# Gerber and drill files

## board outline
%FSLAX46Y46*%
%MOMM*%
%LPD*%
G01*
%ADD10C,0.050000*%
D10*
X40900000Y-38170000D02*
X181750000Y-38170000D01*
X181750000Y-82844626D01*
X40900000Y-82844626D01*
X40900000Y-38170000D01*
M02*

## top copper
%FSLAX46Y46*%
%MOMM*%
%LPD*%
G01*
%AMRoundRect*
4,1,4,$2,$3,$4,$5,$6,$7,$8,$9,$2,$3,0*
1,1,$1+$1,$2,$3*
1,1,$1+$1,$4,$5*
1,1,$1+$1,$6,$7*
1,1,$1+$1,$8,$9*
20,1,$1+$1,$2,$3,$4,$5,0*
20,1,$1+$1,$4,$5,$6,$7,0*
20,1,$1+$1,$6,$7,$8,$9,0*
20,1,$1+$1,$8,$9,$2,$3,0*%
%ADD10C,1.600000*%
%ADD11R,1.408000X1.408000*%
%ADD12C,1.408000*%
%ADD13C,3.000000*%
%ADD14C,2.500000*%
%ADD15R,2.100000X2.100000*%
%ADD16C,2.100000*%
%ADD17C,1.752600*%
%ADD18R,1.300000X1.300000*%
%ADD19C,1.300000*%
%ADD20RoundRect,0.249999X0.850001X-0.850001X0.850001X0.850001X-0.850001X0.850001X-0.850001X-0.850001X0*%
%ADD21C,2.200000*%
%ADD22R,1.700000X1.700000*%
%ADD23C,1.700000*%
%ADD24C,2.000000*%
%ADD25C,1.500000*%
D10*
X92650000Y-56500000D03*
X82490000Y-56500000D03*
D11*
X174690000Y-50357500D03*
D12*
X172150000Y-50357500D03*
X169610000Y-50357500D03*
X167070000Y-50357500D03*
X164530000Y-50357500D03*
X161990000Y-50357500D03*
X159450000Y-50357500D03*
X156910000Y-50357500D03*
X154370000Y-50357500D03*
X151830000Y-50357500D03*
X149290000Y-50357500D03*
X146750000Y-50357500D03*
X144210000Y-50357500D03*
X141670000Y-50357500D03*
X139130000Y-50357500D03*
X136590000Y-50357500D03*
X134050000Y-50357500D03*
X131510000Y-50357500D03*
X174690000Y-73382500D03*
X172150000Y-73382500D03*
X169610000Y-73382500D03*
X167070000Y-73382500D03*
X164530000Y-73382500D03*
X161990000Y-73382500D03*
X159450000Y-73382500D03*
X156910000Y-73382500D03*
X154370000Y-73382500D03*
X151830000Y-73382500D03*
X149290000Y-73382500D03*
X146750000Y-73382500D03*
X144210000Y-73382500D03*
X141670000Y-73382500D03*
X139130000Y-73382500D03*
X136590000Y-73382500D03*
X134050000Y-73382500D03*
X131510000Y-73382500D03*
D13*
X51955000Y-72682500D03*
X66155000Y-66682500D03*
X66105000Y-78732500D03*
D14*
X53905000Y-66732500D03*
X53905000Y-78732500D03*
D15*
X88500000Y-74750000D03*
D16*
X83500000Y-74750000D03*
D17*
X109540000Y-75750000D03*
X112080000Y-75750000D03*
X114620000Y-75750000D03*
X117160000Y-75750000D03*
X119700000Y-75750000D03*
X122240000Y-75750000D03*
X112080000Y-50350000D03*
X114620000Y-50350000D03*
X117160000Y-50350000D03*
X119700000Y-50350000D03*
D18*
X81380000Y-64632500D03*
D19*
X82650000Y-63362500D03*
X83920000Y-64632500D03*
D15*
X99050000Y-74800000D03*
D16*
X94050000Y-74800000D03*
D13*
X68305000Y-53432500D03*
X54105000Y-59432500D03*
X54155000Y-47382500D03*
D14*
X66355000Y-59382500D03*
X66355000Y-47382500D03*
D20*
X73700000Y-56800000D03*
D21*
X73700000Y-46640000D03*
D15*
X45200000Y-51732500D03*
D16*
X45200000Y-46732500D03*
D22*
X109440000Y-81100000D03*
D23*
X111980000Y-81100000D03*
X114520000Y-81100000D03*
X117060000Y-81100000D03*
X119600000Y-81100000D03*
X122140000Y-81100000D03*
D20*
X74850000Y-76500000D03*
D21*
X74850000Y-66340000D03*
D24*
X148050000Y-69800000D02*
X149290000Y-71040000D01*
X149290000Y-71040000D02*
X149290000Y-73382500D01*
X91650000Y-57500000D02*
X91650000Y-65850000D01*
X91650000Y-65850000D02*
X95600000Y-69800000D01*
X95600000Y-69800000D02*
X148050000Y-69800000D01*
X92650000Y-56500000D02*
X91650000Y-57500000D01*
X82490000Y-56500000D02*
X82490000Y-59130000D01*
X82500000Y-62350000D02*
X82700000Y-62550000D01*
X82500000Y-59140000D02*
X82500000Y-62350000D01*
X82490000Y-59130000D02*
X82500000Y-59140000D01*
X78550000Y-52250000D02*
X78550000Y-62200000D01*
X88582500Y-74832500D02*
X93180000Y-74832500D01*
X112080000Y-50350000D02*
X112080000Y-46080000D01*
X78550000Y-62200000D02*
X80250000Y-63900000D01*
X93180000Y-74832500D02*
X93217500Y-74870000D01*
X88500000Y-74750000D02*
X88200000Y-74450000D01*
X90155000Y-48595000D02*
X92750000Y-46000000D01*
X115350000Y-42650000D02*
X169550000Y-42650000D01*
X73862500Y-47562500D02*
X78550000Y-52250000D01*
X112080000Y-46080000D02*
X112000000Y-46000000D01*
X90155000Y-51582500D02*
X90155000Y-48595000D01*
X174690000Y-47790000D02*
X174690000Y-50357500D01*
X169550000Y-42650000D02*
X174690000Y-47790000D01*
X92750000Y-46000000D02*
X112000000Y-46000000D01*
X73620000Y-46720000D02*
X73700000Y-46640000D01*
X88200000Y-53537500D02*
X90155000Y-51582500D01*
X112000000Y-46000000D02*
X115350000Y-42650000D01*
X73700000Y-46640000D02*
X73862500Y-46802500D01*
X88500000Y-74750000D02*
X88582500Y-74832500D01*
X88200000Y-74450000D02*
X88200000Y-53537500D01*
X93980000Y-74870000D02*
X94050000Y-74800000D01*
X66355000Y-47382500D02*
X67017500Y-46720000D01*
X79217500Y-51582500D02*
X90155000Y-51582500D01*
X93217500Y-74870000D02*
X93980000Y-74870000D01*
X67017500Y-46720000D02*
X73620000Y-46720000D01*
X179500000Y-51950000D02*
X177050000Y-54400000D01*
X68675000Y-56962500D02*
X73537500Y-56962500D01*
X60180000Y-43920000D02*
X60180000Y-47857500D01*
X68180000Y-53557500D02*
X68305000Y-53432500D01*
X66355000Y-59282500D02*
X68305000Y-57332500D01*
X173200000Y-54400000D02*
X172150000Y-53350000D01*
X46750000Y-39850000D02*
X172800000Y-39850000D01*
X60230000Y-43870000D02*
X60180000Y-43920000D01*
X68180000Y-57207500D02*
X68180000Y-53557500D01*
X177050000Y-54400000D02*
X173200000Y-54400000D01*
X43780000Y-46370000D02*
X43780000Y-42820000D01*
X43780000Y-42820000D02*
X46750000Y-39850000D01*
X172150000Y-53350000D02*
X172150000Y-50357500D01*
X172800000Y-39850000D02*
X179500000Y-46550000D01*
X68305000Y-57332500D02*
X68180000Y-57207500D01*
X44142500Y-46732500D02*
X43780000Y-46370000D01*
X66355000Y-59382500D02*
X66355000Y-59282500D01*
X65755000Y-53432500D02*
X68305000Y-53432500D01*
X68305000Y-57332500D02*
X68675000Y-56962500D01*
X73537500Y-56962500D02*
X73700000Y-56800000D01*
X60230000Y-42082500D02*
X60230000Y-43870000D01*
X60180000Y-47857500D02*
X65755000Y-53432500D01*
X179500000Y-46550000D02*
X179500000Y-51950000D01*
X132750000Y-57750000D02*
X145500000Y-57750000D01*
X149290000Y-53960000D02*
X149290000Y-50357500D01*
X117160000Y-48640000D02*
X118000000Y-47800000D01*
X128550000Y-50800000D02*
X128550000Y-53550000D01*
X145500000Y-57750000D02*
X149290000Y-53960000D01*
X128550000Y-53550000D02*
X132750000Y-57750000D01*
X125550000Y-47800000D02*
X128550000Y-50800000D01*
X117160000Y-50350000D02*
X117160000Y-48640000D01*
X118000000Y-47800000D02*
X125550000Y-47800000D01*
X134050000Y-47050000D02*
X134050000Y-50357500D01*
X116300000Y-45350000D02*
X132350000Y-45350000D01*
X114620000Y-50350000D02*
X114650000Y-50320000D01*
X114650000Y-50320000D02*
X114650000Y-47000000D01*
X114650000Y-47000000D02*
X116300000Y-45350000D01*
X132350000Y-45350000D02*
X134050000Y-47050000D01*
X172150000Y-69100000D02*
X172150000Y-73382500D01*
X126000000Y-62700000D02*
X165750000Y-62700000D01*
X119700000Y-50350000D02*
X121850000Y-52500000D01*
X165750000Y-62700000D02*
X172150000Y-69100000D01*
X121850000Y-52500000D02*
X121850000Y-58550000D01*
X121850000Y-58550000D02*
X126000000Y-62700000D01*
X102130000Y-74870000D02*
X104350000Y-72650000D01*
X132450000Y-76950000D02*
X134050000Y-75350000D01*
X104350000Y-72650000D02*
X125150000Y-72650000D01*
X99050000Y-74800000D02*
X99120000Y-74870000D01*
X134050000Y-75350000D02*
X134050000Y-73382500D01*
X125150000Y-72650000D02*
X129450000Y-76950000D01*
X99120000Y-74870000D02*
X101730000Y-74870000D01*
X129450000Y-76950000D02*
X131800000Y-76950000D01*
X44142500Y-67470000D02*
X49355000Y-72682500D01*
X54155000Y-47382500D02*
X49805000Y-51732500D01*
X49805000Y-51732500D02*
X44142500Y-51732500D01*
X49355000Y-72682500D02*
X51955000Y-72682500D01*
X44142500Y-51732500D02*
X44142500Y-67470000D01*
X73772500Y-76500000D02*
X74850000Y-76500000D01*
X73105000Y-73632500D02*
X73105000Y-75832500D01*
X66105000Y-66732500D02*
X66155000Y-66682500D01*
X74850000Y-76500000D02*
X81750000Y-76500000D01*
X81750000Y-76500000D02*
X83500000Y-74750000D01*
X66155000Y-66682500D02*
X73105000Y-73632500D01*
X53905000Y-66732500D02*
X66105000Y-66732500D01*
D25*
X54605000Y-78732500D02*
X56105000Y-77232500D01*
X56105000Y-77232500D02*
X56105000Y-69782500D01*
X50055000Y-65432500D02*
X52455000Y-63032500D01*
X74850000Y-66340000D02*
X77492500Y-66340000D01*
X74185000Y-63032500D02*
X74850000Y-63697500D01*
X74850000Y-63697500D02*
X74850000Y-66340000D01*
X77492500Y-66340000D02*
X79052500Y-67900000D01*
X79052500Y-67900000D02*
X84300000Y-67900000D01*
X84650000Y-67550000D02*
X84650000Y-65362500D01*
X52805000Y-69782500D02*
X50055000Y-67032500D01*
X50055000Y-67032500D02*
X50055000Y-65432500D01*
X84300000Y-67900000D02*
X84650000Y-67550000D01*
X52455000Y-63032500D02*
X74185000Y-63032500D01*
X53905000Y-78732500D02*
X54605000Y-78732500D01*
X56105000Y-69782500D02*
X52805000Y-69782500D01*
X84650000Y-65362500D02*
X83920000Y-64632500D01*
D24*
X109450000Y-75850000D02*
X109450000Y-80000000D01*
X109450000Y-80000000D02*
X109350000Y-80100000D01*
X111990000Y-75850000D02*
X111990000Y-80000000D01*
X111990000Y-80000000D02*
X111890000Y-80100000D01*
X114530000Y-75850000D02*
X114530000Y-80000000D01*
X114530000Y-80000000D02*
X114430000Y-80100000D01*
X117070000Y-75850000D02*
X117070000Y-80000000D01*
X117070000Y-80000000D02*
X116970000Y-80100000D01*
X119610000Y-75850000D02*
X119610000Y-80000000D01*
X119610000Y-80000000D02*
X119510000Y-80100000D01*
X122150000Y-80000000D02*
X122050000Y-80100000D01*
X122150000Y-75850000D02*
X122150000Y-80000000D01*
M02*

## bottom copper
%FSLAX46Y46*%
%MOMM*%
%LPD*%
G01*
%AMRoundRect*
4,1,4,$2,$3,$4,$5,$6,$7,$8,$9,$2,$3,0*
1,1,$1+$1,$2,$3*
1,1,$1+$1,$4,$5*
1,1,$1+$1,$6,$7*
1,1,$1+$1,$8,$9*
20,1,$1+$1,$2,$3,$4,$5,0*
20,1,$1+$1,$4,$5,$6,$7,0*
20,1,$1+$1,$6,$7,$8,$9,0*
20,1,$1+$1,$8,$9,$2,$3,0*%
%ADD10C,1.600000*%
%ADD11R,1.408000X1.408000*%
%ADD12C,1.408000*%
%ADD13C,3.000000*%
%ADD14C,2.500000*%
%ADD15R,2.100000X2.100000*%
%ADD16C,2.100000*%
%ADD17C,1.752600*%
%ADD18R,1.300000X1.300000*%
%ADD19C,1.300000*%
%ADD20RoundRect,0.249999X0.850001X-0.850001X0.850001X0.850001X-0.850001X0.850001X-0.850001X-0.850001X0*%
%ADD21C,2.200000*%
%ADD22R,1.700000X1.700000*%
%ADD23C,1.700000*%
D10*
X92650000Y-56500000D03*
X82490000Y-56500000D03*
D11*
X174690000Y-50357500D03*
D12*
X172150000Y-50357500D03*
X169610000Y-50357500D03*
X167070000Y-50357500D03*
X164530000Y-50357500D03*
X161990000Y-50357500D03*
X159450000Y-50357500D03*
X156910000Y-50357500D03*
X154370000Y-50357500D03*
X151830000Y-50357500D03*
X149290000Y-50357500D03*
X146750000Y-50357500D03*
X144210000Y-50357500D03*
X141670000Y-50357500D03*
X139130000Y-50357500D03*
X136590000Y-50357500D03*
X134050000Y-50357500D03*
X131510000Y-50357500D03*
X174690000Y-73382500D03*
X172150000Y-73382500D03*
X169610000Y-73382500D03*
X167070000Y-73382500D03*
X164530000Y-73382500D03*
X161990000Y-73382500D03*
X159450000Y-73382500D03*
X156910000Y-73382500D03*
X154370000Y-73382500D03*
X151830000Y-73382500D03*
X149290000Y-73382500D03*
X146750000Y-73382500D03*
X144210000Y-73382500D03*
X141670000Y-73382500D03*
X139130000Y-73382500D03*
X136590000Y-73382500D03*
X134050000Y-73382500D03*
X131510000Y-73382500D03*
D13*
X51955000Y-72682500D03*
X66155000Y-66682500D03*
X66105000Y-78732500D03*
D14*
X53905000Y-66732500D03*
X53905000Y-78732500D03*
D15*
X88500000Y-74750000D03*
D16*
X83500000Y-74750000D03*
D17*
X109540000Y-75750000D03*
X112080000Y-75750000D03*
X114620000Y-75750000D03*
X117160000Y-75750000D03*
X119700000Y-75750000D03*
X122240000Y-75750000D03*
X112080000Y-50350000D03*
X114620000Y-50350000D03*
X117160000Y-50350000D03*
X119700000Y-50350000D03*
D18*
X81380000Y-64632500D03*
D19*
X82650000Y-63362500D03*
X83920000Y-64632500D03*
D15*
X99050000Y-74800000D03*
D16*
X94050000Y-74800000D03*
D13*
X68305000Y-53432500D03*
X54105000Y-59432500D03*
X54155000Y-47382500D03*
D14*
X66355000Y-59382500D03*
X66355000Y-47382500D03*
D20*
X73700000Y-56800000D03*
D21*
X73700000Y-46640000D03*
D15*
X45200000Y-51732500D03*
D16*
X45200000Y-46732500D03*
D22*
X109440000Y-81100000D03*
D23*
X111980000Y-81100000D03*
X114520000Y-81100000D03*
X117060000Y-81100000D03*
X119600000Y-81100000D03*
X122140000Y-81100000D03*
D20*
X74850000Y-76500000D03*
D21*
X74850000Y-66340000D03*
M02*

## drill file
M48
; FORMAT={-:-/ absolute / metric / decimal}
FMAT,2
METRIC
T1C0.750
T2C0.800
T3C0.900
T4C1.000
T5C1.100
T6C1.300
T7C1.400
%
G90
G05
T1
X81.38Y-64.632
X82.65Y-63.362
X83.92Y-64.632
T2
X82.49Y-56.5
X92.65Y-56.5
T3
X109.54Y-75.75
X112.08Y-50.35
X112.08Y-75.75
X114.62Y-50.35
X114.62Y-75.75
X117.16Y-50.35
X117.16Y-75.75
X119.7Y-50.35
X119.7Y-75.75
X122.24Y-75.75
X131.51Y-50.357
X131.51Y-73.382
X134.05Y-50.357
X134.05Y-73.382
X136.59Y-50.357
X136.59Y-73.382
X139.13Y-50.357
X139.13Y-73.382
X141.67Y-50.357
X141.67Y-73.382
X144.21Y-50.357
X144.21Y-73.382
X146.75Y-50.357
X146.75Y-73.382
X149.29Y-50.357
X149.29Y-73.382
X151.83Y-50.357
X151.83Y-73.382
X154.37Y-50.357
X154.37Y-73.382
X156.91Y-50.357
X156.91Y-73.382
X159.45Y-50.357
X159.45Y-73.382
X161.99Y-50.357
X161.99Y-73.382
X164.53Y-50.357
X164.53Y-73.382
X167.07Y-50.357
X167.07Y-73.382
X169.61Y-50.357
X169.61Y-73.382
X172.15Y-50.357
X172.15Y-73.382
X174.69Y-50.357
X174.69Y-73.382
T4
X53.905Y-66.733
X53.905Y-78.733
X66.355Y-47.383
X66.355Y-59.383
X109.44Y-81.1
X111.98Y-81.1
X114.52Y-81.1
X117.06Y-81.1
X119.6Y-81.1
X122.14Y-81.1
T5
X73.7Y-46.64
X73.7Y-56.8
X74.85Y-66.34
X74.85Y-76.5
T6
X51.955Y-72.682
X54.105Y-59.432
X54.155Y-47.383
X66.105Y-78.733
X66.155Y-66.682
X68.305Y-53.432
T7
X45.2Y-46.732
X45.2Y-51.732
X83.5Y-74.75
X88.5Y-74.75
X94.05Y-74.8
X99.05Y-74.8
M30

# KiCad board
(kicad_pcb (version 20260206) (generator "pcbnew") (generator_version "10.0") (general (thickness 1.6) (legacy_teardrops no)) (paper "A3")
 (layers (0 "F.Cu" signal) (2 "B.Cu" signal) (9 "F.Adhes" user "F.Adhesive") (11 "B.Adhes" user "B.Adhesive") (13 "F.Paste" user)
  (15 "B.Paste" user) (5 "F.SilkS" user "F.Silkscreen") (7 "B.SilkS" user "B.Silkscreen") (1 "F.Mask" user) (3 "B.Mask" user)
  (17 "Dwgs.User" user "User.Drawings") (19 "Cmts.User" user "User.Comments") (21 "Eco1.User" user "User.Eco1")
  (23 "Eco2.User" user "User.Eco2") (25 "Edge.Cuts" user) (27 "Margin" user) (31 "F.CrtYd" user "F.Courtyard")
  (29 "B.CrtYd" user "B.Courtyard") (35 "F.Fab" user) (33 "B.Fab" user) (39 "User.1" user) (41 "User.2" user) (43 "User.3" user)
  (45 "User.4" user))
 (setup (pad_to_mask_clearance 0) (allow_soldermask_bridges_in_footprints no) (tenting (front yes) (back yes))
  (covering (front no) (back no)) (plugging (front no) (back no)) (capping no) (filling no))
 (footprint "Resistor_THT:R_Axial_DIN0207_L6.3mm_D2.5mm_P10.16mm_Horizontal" (layer "F.Cu") (at 92.65 56.5 180)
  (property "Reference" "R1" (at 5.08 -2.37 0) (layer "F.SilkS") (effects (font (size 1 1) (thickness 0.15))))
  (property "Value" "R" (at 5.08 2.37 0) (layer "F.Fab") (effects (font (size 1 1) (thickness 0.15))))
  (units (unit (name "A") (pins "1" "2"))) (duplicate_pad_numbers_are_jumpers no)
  (pad "1" thru_hole circle (at 0 0 180) (size 1.6 1.6) (drill 0.8) (layers "*.Cu" "*.Mask") (remove_unused_layers no) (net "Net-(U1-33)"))
  (pad "2" thru_hole circle (at 10.16 0 180) (size 1.6 1.6) (drill 0.8) (layers "*.Cu" "*.Mask") (remove_unused_layers no)
   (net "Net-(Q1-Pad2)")))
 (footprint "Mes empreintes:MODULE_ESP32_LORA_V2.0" (layer "F.Cu") (at 152.31 61.87 180)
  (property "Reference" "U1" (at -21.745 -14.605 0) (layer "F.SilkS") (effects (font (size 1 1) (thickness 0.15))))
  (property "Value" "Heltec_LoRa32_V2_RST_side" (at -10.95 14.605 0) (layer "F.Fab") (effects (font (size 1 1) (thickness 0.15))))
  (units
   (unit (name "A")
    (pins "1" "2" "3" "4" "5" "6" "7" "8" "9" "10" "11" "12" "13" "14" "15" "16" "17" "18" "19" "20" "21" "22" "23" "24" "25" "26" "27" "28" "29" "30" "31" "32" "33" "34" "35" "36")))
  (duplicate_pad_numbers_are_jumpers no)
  (pad "1" thru_hole rect (at -22.38 11.5125 180) (size 1.408 1.408) (drill 0.9) (layers "*.Cu" "*.Mask") (remove_unused_layers no)
   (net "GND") (solder_mask_margin 0.102))
  (pad "2" thru_hole circle (at -19.84 11.5125 180) (size 1.408 1.408) (drill 0.9) (layers "*.Cu" "*.Mask") (remove_unused_layers no)
   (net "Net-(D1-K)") (solder_mask_margin 0.102))
  (pad "3" thru_hole circle (at -17.3 11.5125 180) (size 1.408 1.408) (drill 0.9) (layers "*.Cu" "*.Mask") (remove_unused_layers no)
   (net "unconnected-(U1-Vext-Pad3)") (solder_mask_margin 0.102))
  (pad "4" thru_hole circle (at -14.76 11.5125 180) (size 1.408 1.408) (drill 0.9) (layers "*.Cu" "*.Mask") (remove_unused_layers no)
   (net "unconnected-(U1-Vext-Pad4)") (solder_mask_margin 0.102))
  (pad "5" thru_hole circle (at -12.22 11.5125 180) (size 1.408 1.408) (drill 0.9) (layers "*.Cu" "*.Mask") (remove_unused_layers no)
   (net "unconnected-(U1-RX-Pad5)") (solder_mask_margin 0.102))
  (pad "6" thru_hole circle (at -9.68 11.5125 180) (size 1.408 1.408) (drill 0.9) (layers "*.Cu" "*.Mask") (remove_unused_layers no)
   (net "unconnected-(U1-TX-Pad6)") (solder_mask_margin 0.102))
  (pad "7" thru_hole circle (at -7.14 11.5125 180) (size 1.408 1.408) (drill 0.9) (layers "*.Cu" "*.Mask") (remove_unused_layers no)
   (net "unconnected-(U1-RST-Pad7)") (solder_mask_margin 0.102))
  (pad "8" thru_hole circle (at -4.6 11.5125 180) (size 1.408 1.408) (drill 0.9) (layers "*.Cu" "*.Mask") (remove_unused_layers no)
   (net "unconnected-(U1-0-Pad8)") (solder_mask_margin 0.102))
  (pad "9" thru_hole circle (at -2.06 11.5125 180) (size 1.408 1.408) (drill 0.9) (layers "*.Cu" "*.Mask") (remove_unused_layers no)
   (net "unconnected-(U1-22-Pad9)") (solder_mask_margin 0.102))
  (pad "10" thru_hole circle (at 0.48 11.5125 180) (size 1.408 1.408) (drill 0.9) (layers "*.Cu" "*.Mask") (remove_unused_layers no)
   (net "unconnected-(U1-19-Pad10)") (solder_mask_margin 0.102))
  (pad "11" thru_hole circle (at 3.02 11.5125 180) (size 1.408 1.408) (drill 0.9) (layers "*.Cu" "*.Mask") (remove_unused_layers no)
   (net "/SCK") (solder_mask_margin 0.102))
  (pad "12" thru_hole circle (at 5.56 11.5125 180) (size 1.408 1.408) (drill 0.9) (layers "*.Cu" "*.Mask") (remove_unused_layers no)
   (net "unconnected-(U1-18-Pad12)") (solder_mask_margin 0.102))
  (pad "13" thru_hole circle (at 8.1 11.5125 180) (size 1.408 1.408) (drill 0.9) (layers "*.Cu" "*.Mask") (remove_unused_layers no)
   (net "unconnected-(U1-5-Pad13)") (solder_mask_margin 0.102))
  (pad "14" thru_hole circle (at 10.64 11.5125 180) (size 1.408 1.408) (drill 0.9) (layers "*.Cu" "*.Mask") (remove_unused_layers no)
   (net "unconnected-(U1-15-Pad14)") (solder_mask_margin 0.102))
  (pad "15" thru_hole circle (at 13.18 11.5125 180) (size 1.408 1.408) (drill 0.9) (layers "*.Cu" "*.Mask") (remove_unused_layers no)
   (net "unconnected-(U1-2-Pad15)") (solder_mask_margin 0.102))
  (pad "16" thru_hole circle (at 15.72 11.5125 180) (size 1.408 1.408) (drill 0.9) (layers "*.Cu" "*.Mask") (remove_unused_layers no)
   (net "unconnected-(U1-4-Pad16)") (solder_mask_margin 0.102))
  (pad "17" thru_hole circle (at 18.26 11.5125 180) (size 1.408 1.408) (drill 0.9) (layers "*.Cu" "*.Mask") (remove_unused_layers no)
   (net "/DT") (solder_mask_margin 0.102))
  (pad "18" thru_hole circle (at 20.8 11.5125 180) (size 1.408 1.408) (drill 0.9) (layers "*.Cu" "*.Mask") (remove_unused_layers no)
   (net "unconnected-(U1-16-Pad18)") (solder_mask_margin 0.102))
  (pad "19" thru_hole circle (at -22.38 -11.5125 180) (size 1.408 1.408) (drill 0.9) (layers "*.Cu" "*.Mask") (remove_unused_layers no)
   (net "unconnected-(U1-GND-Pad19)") (solder_mask_margin 0.102))
  (pad "20" thru_hole circle (at -19.84 -11.5125 180) (size 1.408 1.408) (drill 0.9) (layers "*.Cu" "*.Mask") (remove_unused_layers no)
   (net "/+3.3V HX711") (solder_mask_margin 0.102))
  (pad "21" thru_hole circle (at -17.3 -11.5125 180) (size 1.408 1.408) (drill 0.9) (layers "*.Cu" "*.Mask") (remove_unused_layers no)
   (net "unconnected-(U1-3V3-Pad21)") (solder_mask_margin 0.102))
  (pad "22" thru_hole circle (at -14.76 -11.5125 180) (size 1.408 1.408) (drill 0.9) (layers "*.Cu" "*.Mask") (remove_unused_layers no)
   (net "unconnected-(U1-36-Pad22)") (solder_mask_margin 0.102))
  (pad "23" thru_hole circle (at -12.22 -11.5125 180) (size 1.408 1.408) (drill 0.9) (layers "*.Cu" "*.Mask") (remove_unused_layers no)
   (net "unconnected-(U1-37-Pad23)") (solder_mask_margin 0.102))
  (pad "24" thru_hole circle (at -9.68 -11.5125 180) (size 1.408 1.408) (drill 0.9) (layers "*.Cu" "*.Mask") (remove_unused_layers no)
   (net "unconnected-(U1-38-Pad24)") (solder_mask_margin 0.102))
  (pad "25" thru_hole circle (at -7.14 -11.5125 180) (size 1.408 1.408) (drill 0.9) (layers "*.Cu" "*.Mask") (remove_unused_layers no)
   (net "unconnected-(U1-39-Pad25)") (solder_mask_margin 0.102))
  (pad "26" thru_hole circle (at -4.6 -11.5125 180) (size 1.408 1.408) (drill 0.9) (layers "*.Cu" "*.Mask") (remove_unused_layers no)
   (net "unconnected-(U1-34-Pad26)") (solder_mask_margin 0.102))
  (pad "27" thru_hole circle (at -2.06 -11.5125 180) (size 1.408 1.408) (drill 0.9) (layers "*.Cu" "*.Mask") (remove_unused_layers no)
   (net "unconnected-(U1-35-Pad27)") (solder_mask_margin 0.102))
  (pad "28" thru_hole circle (at 0.48 -11.5125 180) (size 1.408 1.408) (drill 0.9) (layers "*.Cu" "*.Mask") (remove_unused_layers no)
   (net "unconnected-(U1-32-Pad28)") (solder_mask_margin 0.102))
  (pad "29" thru_hole circle (at 3.02 -11.5125 180) (size 1.408 1.408) (drill 0.9) (layers "*.Cu" "*.Mask") (remove_unused_layers no)
   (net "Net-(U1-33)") (solder_mask_margin 0.102))
  (pad "30" thru_hole circle (at 5.56 -11.5125 180) (size 1.408 1.408) (drill 0.9) (layers "*.Cu" "*.Mask") (remove_unused_layers no)
   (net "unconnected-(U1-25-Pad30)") (solder_mask_margin 0.102))
  (pad "31" thru_hole circle (at 8.1 -11.5125 180) (size 1.408 1.408) (drill 0.9) (layers "*.Cu" "*.Mask") (remove_unused_layers no)
   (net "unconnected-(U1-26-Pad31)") (solder_mask_margin 0.102))
  (pad "32" thru_hole circle (at 10.64 -11.5125 180) (size 1.408 1.408) (drill 0.9) (layers "*.Cu" "*.Mask") (remove_unused_layers no)
   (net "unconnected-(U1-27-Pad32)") (solder_mask_margin 0.102))
  (pad "33" thru_hole circle (at 13.18 -11.5125 180) (size 1.408 1.408) (drill 0.9) (layers "*.Cu" "*.Mask") (remove_unused_layers no)
   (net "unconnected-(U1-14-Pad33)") (solder_mask_margin 0.102))
  (pad "34" thru_hole circle (at 15.72 -11.5125 180) (size 1.408 1.408) (drill 0.9) (layers "*.Cu" "*.Mask") (remove_unused_layers no)
   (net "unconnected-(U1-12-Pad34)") (solder_mask_margin 0.102))
  (pad "35" thru_hole circle (at 18.26 -11.5125 180) (size 1.408 1.408) (drill 0.9) (layers "*.Cu" "*.Mask") (remove_unused_layers no)
   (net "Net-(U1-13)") (solder_mask_margin 0.102))
  (pad "36" thru_hole circle (at 20.8 -11.5125 180) (size 1.408 1.408) (drill 0.9) (layers "*.Cu" "*.Mask") (remove_unused_layers no)
   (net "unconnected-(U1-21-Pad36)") (solder_mask_margin 0.102)))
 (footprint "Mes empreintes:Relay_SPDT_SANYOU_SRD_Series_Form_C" (layer "F.Cu") (at 51.955 72.6825)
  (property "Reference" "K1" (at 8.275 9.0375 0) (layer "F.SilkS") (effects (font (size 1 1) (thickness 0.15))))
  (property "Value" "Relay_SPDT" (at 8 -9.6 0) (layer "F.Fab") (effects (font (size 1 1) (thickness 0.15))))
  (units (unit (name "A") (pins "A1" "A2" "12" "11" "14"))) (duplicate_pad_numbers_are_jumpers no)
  (pad "11" thru_hole circle (at 0 0 90) (size 3 3) (drill 1.3) (layers "*.Cu" "*.Mask") (remove_unused_layers no) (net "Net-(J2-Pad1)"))
  (pad "12" thru_hole circle (at 14.2 -6 90) (size 3 3) (drill 1.3) (layers "*.Cu" "*.Mask") (remove_unused_layers no) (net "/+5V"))
  (pad "14" thru_hole circle (at 14.15 6.05 90) (size 3 3) (drill 1.3) (layers "*.Cu" "*.Mask") (remove_unused_layers no)
   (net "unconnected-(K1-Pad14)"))
  (pad "A1" thru_hole circle (at 1.95 -5.95 90) (size 2.5 2.5) (drill 1) (layers "*.Cu" "*.Mask") (remove_unused_layers no) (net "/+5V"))
  (pad "A2" thru_hole circle (at 1.95 6.05 90) (size 2.5 2.5) (drill 1) (layers "*.Cu" "*.Mask") (remove_unused_layers no)
   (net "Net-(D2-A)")))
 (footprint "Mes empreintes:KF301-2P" (layer "F.Cu") (at 86 74.75 180)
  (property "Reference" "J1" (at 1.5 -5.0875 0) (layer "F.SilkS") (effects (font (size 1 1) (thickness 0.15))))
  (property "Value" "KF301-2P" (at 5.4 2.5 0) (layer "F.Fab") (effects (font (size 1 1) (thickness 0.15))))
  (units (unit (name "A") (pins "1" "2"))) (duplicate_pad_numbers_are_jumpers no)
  (pad "1" thru_hole rect (at -2.5 0 180) (size 2.1 2.1) (drill 1.4) (layers "*.Cu" "*.Mask") (remove_unused_layers no) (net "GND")
   (solder_mask_margin 0.102))
  (pad "2" thru_hole circle (at 2.5 0 180) (size 2.1 2.1) (drill 1.4) (layers "*.Cu" "*.Mask") (remove_unused_layers no) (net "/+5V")
   (solder_mask_margin 0.102)))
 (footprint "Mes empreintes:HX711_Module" (layer "F.Cu") (at 109.54 75.75 90)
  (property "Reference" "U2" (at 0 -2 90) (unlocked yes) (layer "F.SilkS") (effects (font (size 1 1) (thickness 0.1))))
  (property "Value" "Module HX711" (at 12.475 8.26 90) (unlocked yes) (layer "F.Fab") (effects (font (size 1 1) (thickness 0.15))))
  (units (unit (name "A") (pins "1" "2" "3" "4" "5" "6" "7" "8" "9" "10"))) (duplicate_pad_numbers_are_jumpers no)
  (pad "1" thru_hole circle (at 0 0 90) (size 1.7526 1.7526) (drill 0.9) (layers "*.Cu" "*.Mask") (remove_unused_layers no)
   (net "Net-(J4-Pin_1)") (solder_mask_margin 0.102))
  (pad "2" thru_hole circle (at 0 2.54 90) (size 1.7526 1.7526) (drill 0.9) (layers "*.Cu" "*.Mask") (remove_unused_layers no)
   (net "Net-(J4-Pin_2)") (solder_mask_margin 0.102))
  (pad "3" thru_hole circle (at 0 5.08 90) (size 1.7526 1.7526) (drill 0.9) (layers "*.Cu" "*.Mask") (remove_unused_layers no)
   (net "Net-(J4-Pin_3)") (solder_mask_margin 0.102))
  (pad "4" thru_hole circle (at 0 7.62 90) (size 1.7526 1.7526) (drill 0.9) (layers "*.Cu" "*.Mask") (remove_unused_layers no)
   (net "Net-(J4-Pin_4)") (solder_mask_margin 0.102))
  (pad "5" thru_hole circle (at 0 10.16 90) (size 1.7526 1.7526) (drill 0.9) (layers "*.Cu" "*.Mask") (remove_unused_layers no)
   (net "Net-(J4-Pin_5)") (solder_mask_margin 0.102))
  (pad "6" thru_hole circle (at 0 12.7 90) (size 1.7526 1.7526) (drill 0.9) (layers "*.Cu" "*.Mask") (remove_unused_layers no)
   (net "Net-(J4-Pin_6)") (solder_mask_margin 0.102))
  (pad "7" thru_hole circle (at 25.4 2.54 90) (size 1.7526 1.7526) (drill 0.9) (layers "*.Cu" "*.Mask") (remove_unused_layers no)
   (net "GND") (solder_mask_margin 0.102))
  (pad "8" thru_hole circle (at 25.4 5.08 90) (size 1.7526 1.7526) (drill 0.9) (layers "*.Cu" "*.Mask") (remove_unused_layers no)
   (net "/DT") (solder_mask_margin 0.102))
  (pad "9" thru_hole circle (at 25.4 7.62 90) (size 1.7526 1.7526) (drill 0.9) (layers "*.Cu" "*.Mask") (remove_unused_layers no)
   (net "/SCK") (solder_mask_margin 0.102))
  (pad "10" thru_hole circle (at 25.4 10.16 90) (size 1.7526 1.7526) (drill 0.9) (layers "*.Cu" "*.Mask") (remove_unused_layers no)
   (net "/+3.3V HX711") (solder_mask_margin 0.102)))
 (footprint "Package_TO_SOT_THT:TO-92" (layer "F.Cu") (at 81.38 64.6325)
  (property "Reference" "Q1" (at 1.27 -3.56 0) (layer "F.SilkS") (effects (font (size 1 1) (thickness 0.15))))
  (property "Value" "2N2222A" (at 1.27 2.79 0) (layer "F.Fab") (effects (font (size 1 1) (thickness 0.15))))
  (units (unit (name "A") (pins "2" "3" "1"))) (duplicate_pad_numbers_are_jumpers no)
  (pad "1" thru_hole rect (at 0 0) (size 1.3 1.3) (drill 0.75) (layers "*.Cu" "*.Mask") (remove_unused_layers no) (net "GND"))
  (pad "2" thru_hole circle (at 1.27 -1.27) (size 1.3 1.3) (drill 0.75) (layers "*.Cu" "*.Mask") (remove_unused_layers no)
   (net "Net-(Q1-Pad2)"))
  (pad "3" thru_hole circle (at 2.54 0) (size 1.3 1.3) (drill 0.75) (layers "*.Cu" "*.Mask") (remove_unused_layers no) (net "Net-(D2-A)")))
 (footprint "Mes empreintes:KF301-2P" (layer "F.Cu") (at 96.55 74.8 180)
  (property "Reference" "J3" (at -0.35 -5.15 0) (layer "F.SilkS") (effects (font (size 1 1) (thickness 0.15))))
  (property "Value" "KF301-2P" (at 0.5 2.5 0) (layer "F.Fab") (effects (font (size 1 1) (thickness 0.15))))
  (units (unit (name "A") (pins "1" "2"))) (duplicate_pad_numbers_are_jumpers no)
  (pad "1" thru_hole rect (at -2.5 0 180) (size 2.1 2.1) (drill 1.4) (layers "*.Cu" "*.Mask") (remove_unused_layers no) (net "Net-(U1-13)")
   (solder_mask_margin 0.102))
  (pad "2" thru_hole circle (at 2.5 0 180) (size 2.1 2.1) (drill 1.4) (layers "*.Cu" "*.Mask") (remove_unused_layers no) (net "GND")
   (solder_mask_margin 0.102)))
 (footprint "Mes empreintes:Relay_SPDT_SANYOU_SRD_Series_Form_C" (layer "F.Cu") (at 68.305 53.4325 180)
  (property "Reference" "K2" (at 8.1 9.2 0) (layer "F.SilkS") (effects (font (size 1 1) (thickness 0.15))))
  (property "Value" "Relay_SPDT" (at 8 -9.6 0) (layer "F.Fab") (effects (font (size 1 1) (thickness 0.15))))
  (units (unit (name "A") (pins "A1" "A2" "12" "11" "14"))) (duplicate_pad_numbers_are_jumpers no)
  (pad "11" thru_hole circle (at 0 0 270) (size 3 3) (drill 1.3) (layers "*.Cu" "*.Mask") (remove_unused_layers no) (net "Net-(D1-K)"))
  (pad "12" thru_hole circle (at 14.2 -6 270) (size 3 3) (drill 1.3) (layers "*.Cu" "*.Mask") (remove_unused_layers no)
   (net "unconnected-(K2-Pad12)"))
  (pad "14" thru_hole circle (at 14.15 6.05 270) (size 3 3) (drill 1.3) (layers "*.Cu" "*.Mask") (remove_unused_layers no)
   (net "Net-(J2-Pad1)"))
  (pad "A1" thru_hole circle (at 1.95 -5.95 270) (size 2.5 2.5) (drill 1) (layers "*.Cu" "*.Mask") (remove_unused_layers no)
   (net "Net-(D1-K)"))
  (pad "A2" thru_hole circle (at 1.95 6.05 270) (size 2.5 2.5) (drill 1) (layers "*.Cu" "*.Mask") (remove_unused_layers no) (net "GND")))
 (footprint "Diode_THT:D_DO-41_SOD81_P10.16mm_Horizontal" (layer "F.Cu") (at 73.7 56.8 90)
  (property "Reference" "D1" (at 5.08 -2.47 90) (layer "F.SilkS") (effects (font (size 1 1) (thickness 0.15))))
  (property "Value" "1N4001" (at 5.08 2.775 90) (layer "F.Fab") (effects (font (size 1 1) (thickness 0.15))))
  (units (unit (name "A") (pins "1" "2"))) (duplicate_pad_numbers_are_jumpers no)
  (pad "1" thru_hole roundrect (at 0 0 90) (size 2.2 2.2) (drill 1.1) (layers "*.Cu" "*.Mask") (remove_unused_layers no)
   (roundrect_rratio 0.113636) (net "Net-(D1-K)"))
  (pad "2" thru_hole circle (at 10.16 0 90) (size 2.2 2.2) (drill 1.1) (layers "*.Cu" "*.Mask") (remove_unused_layers no) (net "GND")))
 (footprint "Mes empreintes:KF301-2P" (layer "F.Cu") (at 45.2 49.2325 90)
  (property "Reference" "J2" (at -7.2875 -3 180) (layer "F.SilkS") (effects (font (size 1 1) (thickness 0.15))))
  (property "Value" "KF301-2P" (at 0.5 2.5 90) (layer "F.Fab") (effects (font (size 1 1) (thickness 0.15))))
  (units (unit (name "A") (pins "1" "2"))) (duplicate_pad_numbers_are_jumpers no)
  (pad "1" thru_hole rect (at -2.5 0 90) (size 2.1 2.1) (drill 1.4) (layers "*.Cu" "*.Mask") (remove_unused_layers no) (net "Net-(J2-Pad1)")
   (solder_mask_margin 0.102))
  (pad "2" thru_hole circle (at 2.5 0 90) (size 2.1 2.1) (drill 1.4) (layers "*.Cu" "*.Mask") (remove_unused_layers no) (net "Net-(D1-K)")
   (solder_mask_margin 0.102)))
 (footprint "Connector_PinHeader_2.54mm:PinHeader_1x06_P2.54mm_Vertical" (layer "F.Cu") (at 109.44 81.1 90)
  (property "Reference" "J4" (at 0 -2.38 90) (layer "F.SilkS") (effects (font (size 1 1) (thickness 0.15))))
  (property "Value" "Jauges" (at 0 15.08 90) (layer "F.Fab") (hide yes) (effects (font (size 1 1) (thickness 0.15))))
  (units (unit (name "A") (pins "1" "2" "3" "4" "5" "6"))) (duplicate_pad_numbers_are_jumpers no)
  (pad "1" thru_hole rect (at 0 0 90) (size 1.7 1.7) (drill 1) (layers "*.Cu" "*.Mask") (remove_unused_layers no) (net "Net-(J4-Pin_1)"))
  (pad "2" thru_hole circle (at 0 2.54 90) (size 1.7 1.7) (drill 1) (layers "*.Cu" "*.Mask") (remove_unused_layers no)
   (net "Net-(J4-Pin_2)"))
  (pad "3" thru_hole circle (at 0 5.08 90) (size 1.7 1.7) (drill 1) (layers "*.Cu" "*.Mask") (remove_unused_layers no)
   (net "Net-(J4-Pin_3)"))
  (pad "4" thru_hole circle (at 0 7.62 90) (size 1.7 1.7) (drill 1) (layers "*.Cu" "*.Mask") (remove_unused_layers no)
   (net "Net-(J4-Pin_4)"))
  (pad "5" thru_hole circle (at 0 10.16 90) (size 1.7 1.7) (drill 1) (layers "*.Cu" "*.Mask") (remove_unused_layers no)
   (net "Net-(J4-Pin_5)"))
  (pad "6" thru_hole circle (at 0 12.7 90) (size 1.7 1.7) (drill 1) (layers "*.Cu" "*.Mask") (remove_unused_layers no)
   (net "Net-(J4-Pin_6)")))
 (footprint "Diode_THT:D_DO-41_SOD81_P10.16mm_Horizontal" (layer "F.Cu") (at 74.85 76.5 90)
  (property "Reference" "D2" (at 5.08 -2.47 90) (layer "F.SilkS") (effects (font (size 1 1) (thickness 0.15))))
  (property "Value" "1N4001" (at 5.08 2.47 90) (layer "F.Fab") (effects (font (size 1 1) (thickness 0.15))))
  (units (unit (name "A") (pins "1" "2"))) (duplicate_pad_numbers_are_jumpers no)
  (pad "1" thru_hole roundrect (at 0 0 90) (size 2.2 2.2) (drill 1.1) (layers "*.Cu" "*.Mask") (remove_unused_layers no)
   (roundrect_rratio 0.113636) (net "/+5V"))
  (pad "2" thru_hole circle (at 10.16 0 90) (size 2.2 2.2) (drill 1.1) (layers "*.Cu" "*.Mask") (remove_unused_layers no) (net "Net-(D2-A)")))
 (gr_rect (start 40.9 38.17) (end 181.75 82.844626) (stroke (width 0.05) (type default)) (fill no) (layer "Edge.Cuts"))
 (segment (start 148.05 69.8) (end 149.29 71.04) (width 2) (layer "F.Cu") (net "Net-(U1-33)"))
 (segment (start 149.29 71.04) (end 149.29 73.3825) (width 2) (layer "F.Cu") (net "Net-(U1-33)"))
 (segment (start 91.65 57.5) (end 91.65 65.85) (width 2) (layer "F.Cu") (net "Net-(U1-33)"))
 (segment (start 91.65 65.85) (end 95.6 69.8) (width 2) (layer "F.Cu") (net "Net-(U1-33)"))
 (segment (start 95.6 69.8) (end 148.05 69.8) (width 2) (layer "F.Cu") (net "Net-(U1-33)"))
 (segment (start 92.65 56.5) (end 91.65 57.5) (width 2) (layer "F.Cu") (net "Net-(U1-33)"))
 (segment (start 82.49 56.5) (end 82.49 59.13) (width 2) (layer "F.Cu") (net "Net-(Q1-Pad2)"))
 (segment (start 82.5 62.35) (end 82.7 62.55) (width 2) (layer "F.Cu") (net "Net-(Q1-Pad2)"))
 (segment (start 82.5 59.14) (end 82.5 62.35) (width 2) (layer "F.Cu") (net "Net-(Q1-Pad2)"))
 (segment (start 82.49 59.13) (end 82.5 59.14) (width 2) (layer "F.Cu") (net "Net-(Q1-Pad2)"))
 (segment (start 78.55 52.25) (end 78.55 62.2) (width 2) (layer "F.Cu") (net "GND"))
 (segment (start 88.5825 74.8325) (end 93.18 74.8325) (width 2) (layer "F.Cu") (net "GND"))
 (segment (start 112.08 50.35) (end 112.08 46.08) (width 2) (layer "F.Cu") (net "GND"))
 (segment (start 78.55 62.2) (end 80.25 63.9) (width 2) (layer "F.Cu") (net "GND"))
 (segment (start 93.18 74.8325) (end 93.2175 74.87) (width 2) (layer "F.Cu") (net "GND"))
 (segment (start 88.5 74.75) (end 88.2 74.45) (width 2) (layer "F.Cu") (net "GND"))
 (segment (start 90.155 48.595) (end 92.75 46) (width 2) (layer "F.Cu") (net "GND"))
 (segment (start 115.35 42.65) (end 169.55 42.65) (width 2) (layer "F.Cu") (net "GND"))
 (segment (start 73.8625 47.5625) (end 78.55 52.25) (width 2) (layer "F.Cu") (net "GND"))
 (segment (start 112.08 46.08) (end 112 46) (width 2) (layer "F.Cu") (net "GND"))
 (segment (start 90.155 51.5825) (end 90.155 48.595) (width 2) (layer "F.Cu") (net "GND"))
 (segment (start 174.69 47.79) (end 174.69 50.3575) (width 2) (layer "F.Cu") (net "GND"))
 (segment (start 169.55 42.65) (end 174.69 47.79) (width 2) (layer "F.Cu") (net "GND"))
 (segment (start 92.75 46) (end 112 46) (width 2) (layer "F.Cu") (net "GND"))
 (segment (start 73.62 46.72) (end 73.7 46.64) (width 2) (layer "F.Cu") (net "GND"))
 (segment (start 88.2 53.5375) (end 90.155 51.5825) (width 2) (layer "F.Cu") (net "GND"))
 (segment (start 112 46) (end 115.35 42.65) (width 2) (layer "F.Cu") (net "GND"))
 (segment (start 73.7 46.64) (end 73.8625 46.8025) (width 2) (layer "F.Cu") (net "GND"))
 (segment (start 88.5 74.75) (end 88.5825 74.8325) (width 2) (layer "F.Cu") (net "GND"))
 (segment (start 88.2 74.45) (end 88.2 53.5375) (width 2) (layer "F.Cu") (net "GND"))
 (segment (start 93.98 74.87) (end 94.05 74.8) (width 2) (layer "F.Cu") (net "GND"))
 (segment (start 66.355 47.3825) (end 67.0175 46.72) (width 2) (layer "F.Cu") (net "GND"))
 (segment (start 79.2175 51.5825) (end 90.155 51.5825) (width 2) (layer "F.Cu") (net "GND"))
 (segment (start 93.2175 74.87) (end 93.98 74.87) (width 2) (layer "F.Cu") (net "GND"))
 (segment (start 67.0175 46.72) (end 73.62 46.72) (width 2) (layer "F.Cu") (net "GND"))
 (segment (start 179.5 51.95) (end 177.05 54.4) (width 2) (layer "F.Cu") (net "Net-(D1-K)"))
 (segment (start 68.675 56.9625) (end 73.5375 56.9625) (width 2) (layer "F.Cu") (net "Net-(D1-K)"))
 (segment (start 60.18 43.92) (end 60.18 47.8575) (width 2) (layer "F.Cu") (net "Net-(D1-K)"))
 (segment (start 68.18 53.5575) (end 68.305 53.4325) (width 2) (layer "F.Cu") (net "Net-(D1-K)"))
 (segment (start 66.355 59.2825) (end 68.305 57.3325) (width 2) (layer "F.Cu") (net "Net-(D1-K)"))
 (segment (start 173.2 54.4) (end 172.15 53.35) (width 2) (layer "F.Cu") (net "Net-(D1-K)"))
 (segment (start 46.75 39.85) (end 172.8 39.85) (width 2) (layer "F.Cu") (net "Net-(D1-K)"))
 (segment (start 60.23 43.87) (end 60.18 43.92) (width 2) (layer "F.Cu") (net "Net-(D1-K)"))
 (segment (start 68.18 57.2075) (end 68.18 53.5575) (width 2) (layer "F.Cu") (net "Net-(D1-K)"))
 (segment (start 177.05 54.4) (end 173.2 54.4) (width 2) (layer "F.Cu") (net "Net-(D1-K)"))
 (segment (start 43.78 46.37) (end 43.78 42.82) (width 2) (layer "F.Cu") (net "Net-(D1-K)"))
 (segment (start 43.78 42.82) (end 46.75 39.85) (width 2) (layer "F.Cu") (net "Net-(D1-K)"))
 (segment (start 172.15 53.35) (end 172.15 50.3575) (width 2) (layer "F.Cu") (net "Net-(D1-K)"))
 (segment (start 172.8 39.85) (end 179.5 46.55) (width 2) (layer "F.Cu") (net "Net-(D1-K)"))
 (segment (start 68.305 57.3325) (end 68.18 57.2075) (width 2) (layer "F.Cu") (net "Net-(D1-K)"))
 (segment (start 44.1425 46.7325) (end 43.78 46.37) (width 2) (layer "F.Cu") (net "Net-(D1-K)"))
 (segment (start 66.355 59.3825) (end 66.355 59.2825) (width 2) (layer "F.Cu") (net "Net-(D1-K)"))
 (segment (start 65.755 53.4325) (end 68.305 53.4325) (width 2) (layer "F.Cu") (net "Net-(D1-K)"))
 (segment (start 68.305 57.3325) (end 68.675 56.9625) (width 2) (layer "F.Cu") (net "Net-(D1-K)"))
 (segment (start 73.5375 56.9625) (end 73.7 56.8) (width 2) (layer "F.Cu") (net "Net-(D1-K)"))
 (segment (start 60.23 42.0825) (end 60.23 43.87) (width 2) (layer "F.Cu") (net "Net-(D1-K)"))
 (segment (start 60.18 47.8575) (end 65.755 53.4325) (width 2) (layer "F.Cu") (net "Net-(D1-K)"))
 (segment (start 179.5 46.55) (end 179.5 51.95) (width 2) (layer "F.Cu") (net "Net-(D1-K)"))
 (segment (start 132.75 57.75) (end 145.5 57.75) (width 2) (layer "F.Cu") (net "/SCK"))
 (segment (start 149.29 53.96) (end 149.29 50.3575) (width 2) (layer "F.Cu") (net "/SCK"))
 (segment (start 117.16 48.64) (end 118 47.8) (width 2) (layer "F.Cu") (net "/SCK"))
 (segment (start 128.55 50.8) (end 128.55 53.55) (width 2) (layer "F.Cu") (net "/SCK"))
 (segment (start 145.5 57.75) (end 149.29 53.96) (width 2) (layer "F.Cu") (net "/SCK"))
 (segment (start 128.55 53.55) (end 132.75 57.75) (width 2) (layer "F.Cu") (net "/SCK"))
 (segment (start 125.55 47.8) (end 128.55 50.8) (width 2) (layer "F.Cu") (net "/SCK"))
 (segment (start 117.16 50.35) (end 117.16 48.64) (width 2) (layer "F.Cu") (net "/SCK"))
 (segment (start 118 47.8) (end 125.55 47.8) (width 2) (layer "F.Cu") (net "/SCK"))
 (segment (start 134.05 47.05) (end 134.05 50.3575) (width 2) (layer "F.Cu") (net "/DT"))
 (segment (start 116.3 45.35) (end 132.35 45.35) (width 2) (layer "F.Cu") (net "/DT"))
 (segment (start 114.62 50.35) (end 114.65 50.32) (width 2) (layer "F.Cu") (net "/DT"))
 (segment (start 114.65 50.32) (end 114.65 47) (width 2) (layer "F.Cu") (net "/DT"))
 (segment (start 114.65 47) (end 116.3 45.35) (width 2) (layer "F.Cu") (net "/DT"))
 (segment (start 132.35 45.35) (end 134.05 47.05) (width 2) (layer "F.Cu") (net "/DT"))
 (segment (start 172.15 69.1) (end 172.15 73.3825) (width 2) (layer "F.Cu") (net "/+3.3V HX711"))
 (segment (start 126 62.7) (end 165.75 62.7) (width 2) (layer "F.Cu") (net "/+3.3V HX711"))
 (segment (start 119.7 50.35) (end 121.85 52.5) (width 2) (layer "F.Cu") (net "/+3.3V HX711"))
 (segment (start 165.75 62.7) (end 172.15 69.1) (width 2) (layer "F.Cu") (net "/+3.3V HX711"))
 (segment (start 121.85 52.5) (end 121.85 58.55) (width 2) (layer "F.Cu") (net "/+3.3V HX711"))
 (segment (start 121.85 58.55) (end 126 62.7) (width 2) (layer "F.Cu") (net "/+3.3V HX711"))
 (segment (start 102.13 74.87) (end 104.35 72.65) (width 2) (layer "F.Cu") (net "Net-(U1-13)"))
 (segment (start 132.45 76.95) (end 134.05 75.35) (width 2) (layer "F.Cu") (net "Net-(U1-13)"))
 (segment (start 104.35 72.65) (end 125.15 72.65) (width 2) (layer "F.Cu") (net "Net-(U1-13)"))
 (segment (start 99.05 74.8) (end 99.12 74.87) (width 2) (layer "F.Cu") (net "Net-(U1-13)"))
 (segment (start 134.05 75.35) (end 134.05 73.3825) (width 2) (layer "F.Cu") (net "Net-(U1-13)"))
 (segment (start 125.15 72.65) (end 129.45 76.95) (width 2) (layer "F.Cu") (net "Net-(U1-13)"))
 (segment (start 99.12 74.87) (end 101.73 74.87) (width 2) (layer "F.Cu") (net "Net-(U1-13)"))
 (segment (start 129.45 76.95) (end 131.8 76.95) (width 2) (layer "F.Cu") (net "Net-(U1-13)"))
 (segment (start 44.1425 67.47) (end 49.355 72.6825) (width 2) (layer "F.Cu") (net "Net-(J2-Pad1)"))
 (segment (start 54.155 47.3825) (end 49.805 51.7325) (width 2) (layer "F.Cu") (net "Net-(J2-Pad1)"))
 (segment (start 49.805 51.7325) (end 44.1425 51.7325) (width 2) (layer "F.Cu") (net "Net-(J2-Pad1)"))
 (segment (start 49.355 72.6825) (end 51.955 72.6825) (width 2) (layer "F.Cu") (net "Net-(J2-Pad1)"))
 (segment (start 44.1425 51.7325) (end 44.1425 67.47) (width 2) (layer "F.Cu") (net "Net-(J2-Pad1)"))
 (segment (start 73.7725 76.5) (end 74.85 76.5) (width 2) (layer "F.Cu") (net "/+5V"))
 (segment (start 73.105 73.6325) (end 73.105 75.8325) (width 2) (layer "F.Cu") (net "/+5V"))
 (segment (start 66.105 66.7325) (end 66.155 66.6825) (width 2) (layer "F.Cu") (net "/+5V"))
 (segment (start 74.85 76.5) (end 81.75 76.5) (width 2) (layer "F.Cu") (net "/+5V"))
 (segment (start 81.75 76.5) (end 83.5 74.75) (width 2) (layer "F.Cu") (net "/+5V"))
 (segment (start 66.155 66.6825) (end 73.105 73.6325) (width 2) (layer "F.Cu") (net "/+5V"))
 (segment (start 53.905 66.7325) (end 66.105 66.7325) (width 2) (layer "F.Cu") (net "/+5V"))
 (segment (start 54.605 78.7325) (end 56.105 77.2325) (width 1.5) (layer "F.Cu") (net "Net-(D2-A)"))
 (segment (start 56.105 77.2325) (end 56.105 69.7825) (width 1.5) (layer "F.Cu") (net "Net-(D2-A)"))
 (segment (start 50.055 65.4325) (end 52.455 63.0325) (width 1.5) (layer "F.Cu") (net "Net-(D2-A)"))
 (segment (start 74.85 66.34) (end 77.4925 66.34) (width 1.5) (layer "F.Cu") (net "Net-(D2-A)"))
 (segment (start 74.185 63.0325) (end 74.85 63.6975) (width 1.5) (layer "F.Cu") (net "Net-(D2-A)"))
 (segment (start 74.85 63.6975) (end 74.85 66.34) (width 1.5) (layer "F.Cu") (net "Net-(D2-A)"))
 (segment (start 77.4925 66.34) (end 79.0525 67.9) (width 1.5) (layer "F.Cu") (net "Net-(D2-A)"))
 (segment (start 79.0525 67.9) (end 84.3 67.9) (width 1.5) (layer "F.Cu") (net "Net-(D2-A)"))
 (segment (start 84.65 67.55) (end 84.65 65.3625) (width 1.5) (layer "F.Cu") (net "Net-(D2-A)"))
 (segment (start 52.805 69.7825) (end 50.055 67.0325) (width 1.5) (layer "F.Cu") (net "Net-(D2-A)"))
 (segment (start 50.055 67.0325) (end 50.055 65.4325) (width 1.5) (layer "F.Cu") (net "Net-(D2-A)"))
 (segment (start 84.3 67.9) (end 84.65 67.55) (width 1.5) (layer "F.Cu") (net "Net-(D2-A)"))
 (segment (start 52.455 63.0325) (end 74.185 63.0325) (width 1.5) (layer "F.Cu") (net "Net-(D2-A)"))
 (segment (start 53.905 78.7325) (end 54.605 78.7325) (width 1.5) (layer "F.Cu") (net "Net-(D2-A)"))
 (segment (start 56.105 69.7825) (end 52.805 69.7825) (width 1.5) (layer "F.Cu") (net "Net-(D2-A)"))
 (segment (start 84.65 65.3625) (end 83.92 64.6325) (width 1.5) (layer "F.Cu") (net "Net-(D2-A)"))
 (segment (start 109.45 75.85) (end 109.45 80) (width 2) (layer "F.Cu") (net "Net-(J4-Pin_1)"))
 (segment (start 109.45 80) (end 109.35 80.1) (width 2) (layer "F.Cu") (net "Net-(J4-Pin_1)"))
 (segment (start 111.99 75.85) (end 111.99 80) (width 2) (layer "F.Cu") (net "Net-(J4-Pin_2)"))
 (segment (start 111.99 80) (end 111.89 80.1) (width 2) (layer "F.Cu") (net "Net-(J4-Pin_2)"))
 (segment (start 114.53 75.85) (end 114.53 80) (width 2) (layer "F.Cu") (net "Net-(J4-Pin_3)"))
 (segment (start 114.53 80) (end 114.43 80.1) (width 2) (layer "F.Cu") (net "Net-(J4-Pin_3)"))
 (segment (start 117.07 75.85) (end 117.07 80) (width 2) (layer "F.Cu") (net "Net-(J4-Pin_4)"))
 (segment (start 117.07 80) (end 116.97 80.1) (width 2) (layer "F.Cu") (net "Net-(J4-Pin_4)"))
 (segment (start 119.61 75.85) (end 119.61 80) (width 2) (layer "F.Cu") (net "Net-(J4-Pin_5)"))
 (segment (start 119.61 80) (end 119.51 80.1) (width 2) (layer "F.Cu") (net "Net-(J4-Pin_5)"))
 (segment (start 122.15 80) (end 122.05 80.1) (width 2) (layer "F.Cu") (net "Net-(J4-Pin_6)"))
 (segment (start 122.15 75.85) (end 122.15 80) (width 2) (layer "F.Cu") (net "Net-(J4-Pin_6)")))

